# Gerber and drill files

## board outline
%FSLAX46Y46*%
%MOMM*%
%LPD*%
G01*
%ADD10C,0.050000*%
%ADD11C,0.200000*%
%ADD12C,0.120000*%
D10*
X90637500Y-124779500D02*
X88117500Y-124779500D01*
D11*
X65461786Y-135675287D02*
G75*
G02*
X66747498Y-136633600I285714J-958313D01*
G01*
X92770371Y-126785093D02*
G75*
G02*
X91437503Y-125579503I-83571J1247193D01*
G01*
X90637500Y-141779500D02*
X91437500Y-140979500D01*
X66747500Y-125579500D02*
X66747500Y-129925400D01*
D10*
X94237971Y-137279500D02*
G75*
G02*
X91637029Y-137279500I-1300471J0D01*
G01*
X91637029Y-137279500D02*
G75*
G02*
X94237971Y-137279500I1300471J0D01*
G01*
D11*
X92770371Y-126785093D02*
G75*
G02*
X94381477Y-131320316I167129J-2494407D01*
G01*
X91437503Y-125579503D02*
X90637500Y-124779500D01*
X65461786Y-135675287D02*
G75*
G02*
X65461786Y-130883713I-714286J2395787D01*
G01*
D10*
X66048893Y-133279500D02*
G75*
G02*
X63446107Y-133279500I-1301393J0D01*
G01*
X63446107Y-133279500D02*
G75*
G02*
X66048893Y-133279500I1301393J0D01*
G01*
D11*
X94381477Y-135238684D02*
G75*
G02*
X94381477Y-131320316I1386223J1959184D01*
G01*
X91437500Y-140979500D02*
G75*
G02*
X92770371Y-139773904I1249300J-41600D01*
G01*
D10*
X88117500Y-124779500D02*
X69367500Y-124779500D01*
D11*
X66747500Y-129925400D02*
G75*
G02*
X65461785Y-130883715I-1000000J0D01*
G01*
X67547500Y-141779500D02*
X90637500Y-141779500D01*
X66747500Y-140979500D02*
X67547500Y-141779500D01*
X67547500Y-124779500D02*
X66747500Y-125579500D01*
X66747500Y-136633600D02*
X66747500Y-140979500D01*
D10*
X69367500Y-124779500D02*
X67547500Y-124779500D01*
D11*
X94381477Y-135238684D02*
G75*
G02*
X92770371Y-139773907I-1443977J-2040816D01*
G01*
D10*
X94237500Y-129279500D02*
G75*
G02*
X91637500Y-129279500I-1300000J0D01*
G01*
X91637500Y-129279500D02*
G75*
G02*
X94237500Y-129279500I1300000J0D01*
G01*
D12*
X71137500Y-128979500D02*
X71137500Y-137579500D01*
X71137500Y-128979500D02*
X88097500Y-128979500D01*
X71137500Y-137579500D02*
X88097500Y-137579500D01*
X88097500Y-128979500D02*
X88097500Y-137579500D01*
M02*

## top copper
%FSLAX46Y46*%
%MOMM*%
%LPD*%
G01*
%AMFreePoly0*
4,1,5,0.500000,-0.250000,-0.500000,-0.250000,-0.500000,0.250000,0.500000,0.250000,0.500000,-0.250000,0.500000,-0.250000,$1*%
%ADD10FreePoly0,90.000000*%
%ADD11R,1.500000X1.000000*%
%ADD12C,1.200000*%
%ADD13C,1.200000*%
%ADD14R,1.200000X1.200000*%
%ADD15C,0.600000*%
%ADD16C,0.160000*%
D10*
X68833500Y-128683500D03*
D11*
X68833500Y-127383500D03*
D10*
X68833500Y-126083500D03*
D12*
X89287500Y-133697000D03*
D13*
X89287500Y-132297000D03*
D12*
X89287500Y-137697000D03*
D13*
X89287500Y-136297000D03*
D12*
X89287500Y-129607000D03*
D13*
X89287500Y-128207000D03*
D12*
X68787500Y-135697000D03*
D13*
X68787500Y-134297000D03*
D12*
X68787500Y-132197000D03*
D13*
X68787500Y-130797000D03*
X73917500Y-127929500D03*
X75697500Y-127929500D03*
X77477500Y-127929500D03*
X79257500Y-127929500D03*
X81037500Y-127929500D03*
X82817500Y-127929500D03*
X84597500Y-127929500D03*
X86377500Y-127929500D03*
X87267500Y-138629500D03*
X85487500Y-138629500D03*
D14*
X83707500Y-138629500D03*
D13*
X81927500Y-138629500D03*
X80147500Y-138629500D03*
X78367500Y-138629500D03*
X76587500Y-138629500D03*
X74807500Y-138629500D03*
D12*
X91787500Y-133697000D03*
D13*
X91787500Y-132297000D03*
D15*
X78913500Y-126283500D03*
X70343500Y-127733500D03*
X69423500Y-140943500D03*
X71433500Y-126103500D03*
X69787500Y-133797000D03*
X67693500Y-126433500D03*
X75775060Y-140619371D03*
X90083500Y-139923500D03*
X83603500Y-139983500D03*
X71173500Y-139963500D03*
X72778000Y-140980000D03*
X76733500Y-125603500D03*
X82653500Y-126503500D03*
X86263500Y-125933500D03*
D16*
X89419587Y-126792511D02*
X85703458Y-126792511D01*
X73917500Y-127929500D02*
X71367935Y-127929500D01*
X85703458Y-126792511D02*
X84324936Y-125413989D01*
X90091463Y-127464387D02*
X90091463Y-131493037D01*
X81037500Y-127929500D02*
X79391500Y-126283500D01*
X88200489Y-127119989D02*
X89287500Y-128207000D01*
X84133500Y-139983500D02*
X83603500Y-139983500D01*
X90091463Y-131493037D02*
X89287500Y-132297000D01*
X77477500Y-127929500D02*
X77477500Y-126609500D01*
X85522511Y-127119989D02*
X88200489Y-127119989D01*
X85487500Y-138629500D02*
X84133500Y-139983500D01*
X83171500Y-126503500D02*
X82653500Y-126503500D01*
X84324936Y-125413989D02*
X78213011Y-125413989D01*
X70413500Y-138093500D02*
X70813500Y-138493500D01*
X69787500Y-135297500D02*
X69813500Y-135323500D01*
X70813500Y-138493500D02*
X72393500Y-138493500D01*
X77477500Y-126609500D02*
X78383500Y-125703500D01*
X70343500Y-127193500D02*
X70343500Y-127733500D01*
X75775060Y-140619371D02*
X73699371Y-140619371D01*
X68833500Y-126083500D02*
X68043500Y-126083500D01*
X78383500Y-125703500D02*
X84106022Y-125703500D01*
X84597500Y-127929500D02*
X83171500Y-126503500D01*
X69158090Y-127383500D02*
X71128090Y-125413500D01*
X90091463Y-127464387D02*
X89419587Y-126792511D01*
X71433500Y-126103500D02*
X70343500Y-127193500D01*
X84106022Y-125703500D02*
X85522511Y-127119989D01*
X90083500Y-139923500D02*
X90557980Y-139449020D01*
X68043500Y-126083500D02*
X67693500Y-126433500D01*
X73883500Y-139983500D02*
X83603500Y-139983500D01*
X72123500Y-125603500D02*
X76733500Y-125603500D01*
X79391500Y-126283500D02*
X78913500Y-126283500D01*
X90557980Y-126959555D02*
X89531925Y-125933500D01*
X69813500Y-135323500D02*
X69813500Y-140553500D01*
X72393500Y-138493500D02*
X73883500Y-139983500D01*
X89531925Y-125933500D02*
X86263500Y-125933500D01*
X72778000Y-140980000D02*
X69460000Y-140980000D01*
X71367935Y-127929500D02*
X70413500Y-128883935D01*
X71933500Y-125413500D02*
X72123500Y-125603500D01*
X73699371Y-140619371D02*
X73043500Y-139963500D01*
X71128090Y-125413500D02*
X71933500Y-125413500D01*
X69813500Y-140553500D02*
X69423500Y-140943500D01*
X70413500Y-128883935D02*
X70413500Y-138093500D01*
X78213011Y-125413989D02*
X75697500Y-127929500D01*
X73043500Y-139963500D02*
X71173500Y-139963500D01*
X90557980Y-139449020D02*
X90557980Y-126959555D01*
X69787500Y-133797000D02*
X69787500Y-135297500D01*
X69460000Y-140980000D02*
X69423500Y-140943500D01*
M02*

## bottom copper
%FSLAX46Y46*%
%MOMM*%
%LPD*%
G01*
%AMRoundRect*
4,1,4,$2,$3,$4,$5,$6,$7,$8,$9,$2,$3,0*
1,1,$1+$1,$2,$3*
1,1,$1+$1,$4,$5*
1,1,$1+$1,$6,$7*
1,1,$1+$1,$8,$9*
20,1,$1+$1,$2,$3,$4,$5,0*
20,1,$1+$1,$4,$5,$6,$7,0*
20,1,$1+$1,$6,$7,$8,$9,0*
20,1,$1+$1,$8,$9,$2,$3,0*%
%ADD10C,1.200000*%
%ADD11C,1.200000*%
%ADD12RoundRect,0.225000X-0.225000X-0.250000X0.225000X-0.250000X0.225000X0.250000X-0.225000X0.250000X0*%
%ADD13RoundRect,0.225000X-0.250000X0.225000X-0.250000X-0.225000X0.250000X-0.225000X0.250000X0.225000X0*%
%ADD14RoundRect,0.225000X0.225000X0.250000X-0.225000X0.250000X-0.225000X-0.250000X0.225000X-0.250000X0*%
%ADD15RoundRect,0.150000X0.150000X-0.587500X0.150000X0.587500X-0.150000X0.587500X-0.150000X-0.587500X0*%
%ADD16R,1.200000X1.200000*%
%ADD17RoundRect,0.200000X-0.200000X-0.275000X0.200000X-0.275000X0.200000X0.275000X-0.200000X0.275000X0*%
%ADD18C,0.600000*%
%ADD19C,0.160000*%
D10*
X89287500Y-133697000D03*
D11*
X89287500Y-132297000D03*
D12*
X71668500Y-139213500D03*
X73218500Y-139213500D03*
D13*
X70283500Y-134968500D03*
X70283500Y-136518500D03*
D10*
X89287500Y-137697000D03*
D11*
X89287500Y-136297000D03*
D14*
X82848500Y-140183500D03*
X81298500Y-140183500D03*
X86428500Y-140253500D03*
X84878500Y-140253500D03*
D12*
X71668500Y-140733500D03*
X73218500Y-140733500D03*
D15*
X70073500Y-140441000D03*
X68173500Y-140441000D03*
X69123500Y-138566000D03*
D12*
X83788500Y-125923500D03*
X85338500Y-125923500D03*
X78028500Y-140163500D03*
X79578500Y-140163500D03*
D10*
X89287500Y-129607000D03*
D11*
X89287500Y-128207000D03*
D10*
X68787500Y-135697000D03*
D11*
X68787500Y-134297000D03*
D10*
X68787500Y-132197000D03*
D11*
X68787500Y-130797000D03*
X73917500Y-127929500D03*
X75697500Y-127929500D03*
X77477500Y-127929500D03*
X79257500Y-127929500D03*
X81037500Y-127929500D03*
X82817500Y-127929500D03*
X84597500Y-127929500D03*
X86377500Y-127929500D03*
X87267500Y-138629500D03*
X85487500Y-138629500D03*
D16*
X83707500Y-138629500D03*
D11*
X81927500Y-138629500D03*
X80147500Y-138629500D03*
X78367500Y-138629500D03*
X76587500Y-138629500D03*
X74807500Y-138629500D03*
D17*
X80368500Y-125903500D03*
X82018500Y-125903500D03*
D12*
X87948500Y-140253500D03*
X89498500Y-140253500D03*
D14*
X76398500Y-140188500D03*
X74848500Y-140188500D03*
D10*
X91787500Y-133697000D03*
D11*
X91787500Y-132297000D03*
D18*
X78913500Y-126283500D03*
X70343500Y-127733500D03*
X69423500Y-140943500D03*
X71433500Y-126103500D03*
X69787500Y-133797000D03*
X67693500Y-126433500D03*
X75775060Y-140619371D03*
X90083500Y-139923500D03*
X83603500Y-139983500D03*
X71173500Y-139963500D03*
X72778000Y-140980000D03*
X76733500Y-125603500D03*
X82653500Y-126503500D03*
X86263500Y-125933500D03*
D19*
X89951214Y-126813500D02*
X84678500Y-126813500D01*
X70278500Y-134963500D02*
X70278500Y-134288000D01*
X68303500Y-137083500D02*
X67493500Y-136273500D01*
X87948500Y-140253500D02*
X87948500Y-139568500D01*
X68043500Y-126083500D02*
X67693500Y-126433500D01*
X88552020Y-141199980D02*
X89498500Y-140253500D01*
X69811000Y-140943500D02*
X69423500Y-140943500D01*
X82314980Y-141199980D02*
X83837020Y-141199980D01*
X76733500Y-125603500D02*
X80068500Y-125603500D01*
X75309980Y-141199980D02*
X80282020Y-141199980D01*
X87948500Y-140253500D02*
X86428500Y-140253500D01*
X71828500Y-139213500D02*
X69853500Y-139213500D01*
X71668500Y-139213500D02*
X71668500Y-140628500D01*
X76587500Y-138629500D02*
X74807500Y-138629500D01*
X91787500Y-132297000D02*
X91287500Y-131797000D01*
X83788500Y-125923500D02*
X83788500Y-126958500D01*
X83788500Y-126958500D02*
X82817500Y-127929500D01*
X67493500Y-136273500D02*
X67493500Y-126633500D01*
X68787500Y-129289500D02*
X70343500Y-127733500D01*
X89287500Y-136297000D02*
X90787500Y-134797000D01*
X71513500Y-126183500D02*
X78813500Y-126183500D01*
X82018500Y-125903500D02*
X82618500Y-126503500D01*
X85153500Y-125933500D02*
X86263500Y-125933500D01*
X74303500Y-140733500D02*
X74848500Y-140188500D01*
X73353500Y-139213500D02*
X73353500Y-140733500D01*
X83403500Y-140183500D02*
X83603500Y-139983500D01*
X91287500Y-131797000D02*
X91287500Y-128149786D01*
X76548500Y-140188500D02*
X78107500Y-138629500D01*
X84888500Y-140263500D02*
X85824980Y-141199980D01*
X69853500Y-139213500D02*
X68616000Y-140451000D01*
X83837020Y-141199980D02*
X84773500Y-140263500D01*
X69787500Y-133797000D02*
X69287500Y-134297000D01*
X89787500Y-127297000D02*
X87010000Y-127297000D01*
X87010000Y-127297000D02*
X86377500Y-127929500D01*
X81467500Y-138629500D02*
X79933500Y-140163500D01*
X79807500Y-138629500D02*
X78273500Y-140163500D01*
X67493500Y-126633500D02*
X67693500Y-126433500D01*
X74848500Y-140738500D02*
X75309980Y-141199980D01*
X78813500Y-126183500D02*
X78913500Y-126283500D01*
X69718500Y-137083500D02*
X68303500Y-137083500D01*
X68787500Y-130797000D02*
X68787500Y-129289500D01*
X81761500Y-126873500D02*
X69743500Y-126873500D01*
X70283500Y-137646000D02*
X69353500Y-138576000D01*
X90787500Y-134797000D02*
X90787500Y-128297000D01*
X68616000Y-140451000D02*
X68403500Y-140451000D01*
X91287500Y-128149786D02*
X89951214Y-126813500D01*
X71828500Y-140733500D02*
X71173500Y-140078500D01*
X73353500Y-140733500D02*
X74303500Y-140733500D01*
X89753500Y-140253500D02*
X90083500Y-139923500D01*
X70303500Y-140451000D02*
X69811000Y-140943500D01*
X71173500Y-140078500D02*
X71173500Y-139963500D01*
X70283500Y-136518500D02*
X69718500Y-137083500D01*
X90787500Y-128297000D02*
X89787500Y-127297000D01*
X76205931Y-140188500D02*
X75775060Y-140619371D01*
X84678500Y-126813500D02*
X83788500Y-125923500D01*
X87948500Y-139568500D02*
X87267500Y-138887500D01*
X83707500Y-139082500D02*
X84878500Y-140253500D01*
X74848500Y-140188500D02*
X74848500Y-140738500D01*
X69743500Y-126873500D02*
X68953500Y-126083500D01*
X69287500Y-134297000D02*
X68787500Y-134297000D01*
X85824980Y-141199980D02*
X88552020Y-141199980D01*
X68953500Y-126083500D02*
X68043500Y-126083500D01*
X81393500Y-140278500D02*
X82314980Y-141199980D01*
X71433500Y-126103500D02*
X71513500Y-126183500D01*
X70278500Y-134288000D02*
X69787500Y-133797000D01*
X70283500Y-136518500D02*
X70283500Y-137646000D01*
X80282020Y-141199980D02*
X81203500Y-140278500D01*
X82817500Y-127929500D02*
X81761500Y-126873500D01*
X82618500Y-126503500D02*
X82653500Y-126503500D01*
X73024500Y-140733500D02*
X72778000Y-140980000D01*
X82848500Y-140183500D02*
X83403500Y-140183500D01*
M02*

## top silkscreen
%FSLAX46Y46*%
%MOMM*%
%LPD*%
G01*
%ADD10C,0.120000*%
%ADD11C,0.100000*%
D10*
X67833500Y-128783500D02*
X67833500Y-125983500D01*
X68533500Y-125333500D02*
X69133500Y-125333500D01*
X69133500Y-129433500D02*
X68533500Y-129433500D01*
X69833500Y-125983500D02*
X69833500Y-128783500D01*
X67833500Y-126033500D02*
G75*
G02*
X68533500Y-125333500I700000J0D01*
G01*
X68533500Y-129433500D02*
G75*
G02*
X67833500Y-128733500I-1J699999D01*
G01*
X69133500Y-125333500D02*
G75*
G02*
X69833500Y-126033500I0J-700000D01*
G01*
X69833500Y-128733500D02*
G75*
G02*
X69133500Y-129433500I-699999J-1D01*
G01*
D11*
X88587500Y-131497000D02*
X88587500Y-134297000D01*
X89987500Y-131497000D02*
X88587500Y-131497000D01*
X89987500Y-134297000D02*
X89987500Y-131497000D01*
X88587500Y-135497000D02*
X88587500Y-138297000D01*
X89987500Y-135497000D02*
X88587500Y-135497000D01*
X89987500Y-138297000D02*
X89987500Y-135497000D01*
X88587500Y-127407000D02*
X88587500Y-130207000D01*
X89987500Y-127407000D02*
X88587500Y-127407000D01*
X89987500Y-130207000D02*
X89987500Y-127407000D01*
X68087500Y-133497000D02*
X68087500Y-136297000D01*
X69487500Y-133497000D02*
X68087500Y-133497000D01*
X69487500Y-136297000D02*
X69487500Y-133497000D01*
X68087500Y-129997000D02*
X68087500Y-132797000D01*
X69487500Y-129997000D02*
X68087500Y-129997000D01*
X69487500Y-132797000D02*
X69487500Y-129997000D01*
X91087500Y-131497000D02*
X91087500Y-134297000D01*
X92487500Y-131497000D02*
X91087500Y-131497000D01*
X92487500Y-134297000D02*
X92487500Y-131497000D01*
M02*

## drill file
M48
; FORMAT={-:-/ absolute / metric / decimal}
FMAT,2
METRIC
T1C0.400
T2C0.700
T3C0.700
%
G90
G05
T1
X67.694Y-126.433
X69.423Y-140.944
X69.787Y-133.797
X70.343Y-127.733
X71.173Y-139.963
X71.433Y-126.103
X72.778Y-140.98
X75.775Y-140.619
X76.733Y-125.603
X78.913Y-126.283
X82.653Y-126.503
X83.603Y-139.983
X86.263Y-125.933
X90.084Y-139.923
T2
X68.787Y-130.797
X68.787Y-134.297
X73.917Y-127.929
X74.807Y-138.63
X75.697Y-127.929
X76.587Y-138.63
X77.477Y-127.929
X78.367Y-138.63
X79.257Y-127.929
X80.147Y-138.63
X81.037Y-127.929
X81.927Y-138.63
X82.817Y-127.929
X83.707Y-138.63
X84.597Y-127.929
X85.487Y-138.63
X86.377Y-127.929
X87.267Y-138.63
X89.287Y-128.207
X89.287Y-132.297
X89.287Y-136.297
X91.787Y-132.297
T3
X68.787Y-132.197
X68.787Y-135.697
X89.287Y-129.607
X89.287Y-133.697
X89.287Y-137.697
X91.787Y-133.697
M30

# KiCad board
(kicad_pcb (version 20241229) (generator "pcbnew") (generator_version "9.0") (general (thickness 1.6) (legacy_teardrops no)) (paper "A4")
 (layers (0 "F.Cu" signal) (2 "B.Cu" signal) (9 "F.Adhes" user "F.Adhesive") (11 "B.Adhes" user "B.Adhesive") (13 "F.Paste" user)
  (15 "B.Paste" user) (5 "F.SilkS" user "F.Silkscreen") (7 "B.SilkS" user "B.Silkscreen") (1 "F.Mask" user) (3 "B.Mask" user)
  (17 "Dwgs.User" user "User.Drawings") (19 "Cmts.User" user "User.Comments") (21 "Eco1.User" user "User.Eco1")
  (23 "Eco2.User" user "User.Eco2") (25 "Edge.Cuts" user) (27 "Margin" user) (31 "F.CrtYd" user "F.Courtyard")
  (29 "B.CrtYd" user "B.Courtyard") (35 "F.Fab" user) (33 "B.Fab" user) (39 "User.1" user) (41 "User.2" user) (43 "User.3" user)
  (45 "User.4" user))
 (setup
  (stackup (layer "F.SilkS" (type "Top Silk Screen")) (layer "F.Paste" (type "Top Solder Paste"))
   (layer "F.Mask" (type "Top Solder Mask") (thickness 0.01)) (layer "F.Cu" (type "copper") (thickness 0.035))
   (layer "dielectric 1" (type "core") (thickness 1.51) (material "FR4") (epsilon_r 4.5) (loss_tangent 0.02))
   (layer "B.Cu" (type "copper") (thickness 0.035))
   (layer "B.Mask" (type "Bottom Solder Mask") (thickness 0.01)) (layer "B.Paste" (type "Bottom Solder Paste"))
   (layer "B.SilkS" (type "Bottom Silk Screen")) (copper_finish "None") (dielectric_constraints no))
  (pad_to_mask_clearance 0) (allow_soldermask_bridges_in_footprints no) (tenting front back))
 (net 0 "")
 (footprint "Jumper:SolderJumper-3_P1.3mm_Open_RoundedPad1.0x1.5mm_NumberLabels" (layer "F.Cu") (at 68.8335 127.3835 90)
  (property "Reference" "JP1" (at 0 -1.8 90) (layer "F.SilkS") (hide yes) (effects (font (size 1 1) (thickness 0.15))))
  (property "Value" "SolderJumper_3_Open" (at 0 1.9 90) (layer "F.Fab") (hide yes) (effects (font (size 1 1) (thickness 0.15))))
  (fp_line (start -1.4 -1) (end 1.4 -1) (stroke (width 0.12) (type solid)) (layer "F.SilkS"))
  (fp_line (start 2.05 -0.3) (end 2.05 0.3) (stroke (width 0.12) (type solid)) (layer "F.SilkS"))
  (fp_line (start -2.05 0.3) (end -2.05 -0.3) (stroke (width 0.12) (type solid)) (layer "F.SilkS"))
  (fp_line (start 1.4 1) (end -1.4 1) (stroke (width 0.12) (type solid)) (layer "F.SilkS"))
  (fp_arc (start 1.35 -1) (mid 1.844975 -0.794975) (end 2.05 -0.3) (stroke (width 0.12) (type solid)) (layer "F.SilkS"))
  (fp_arc (start -2.05 -0.3) (mid -1.844975 -0.794975) (end -1.35 -1) (stroke (width 0.12) (type solid)) (layer "F.SilkS"))
  (fp_arc (start 2.05 0.3) (mid 1.844975 0.794975) (end 1.35 1) (stroke (width 0.12) (type solid)) (layer "F.SilkS"))
  (fp_arc (start -1.35 1) (mid -1.844975 0.794975) (end -2.05 0.3) (stroke (width 0.12) (type solid)) (layer "F.SilkS"))
  (pad "1" smd custom (at -1.3 0 90) (size 1 0.5) (layers "F.Cu" "F.Mask") (zone_connect 2) (options (clearance outline) (anchor rect))
   (primitives))
  (pad "2" smd rect (at 0 0 90) (size 1 1.5) (layers "F.Cu" "F.Mask"))
  (pad "3" smd custom (at 1.3 0 90) (size 1 0.5) (layers "F.Cu" "F.Mask") (zone_connect 2) (options (clearance outline) (anchor rect))
   (primitives)))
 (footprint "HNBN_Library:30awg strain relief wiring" (layer "B.Cu") (at 89.2875 132.297 90)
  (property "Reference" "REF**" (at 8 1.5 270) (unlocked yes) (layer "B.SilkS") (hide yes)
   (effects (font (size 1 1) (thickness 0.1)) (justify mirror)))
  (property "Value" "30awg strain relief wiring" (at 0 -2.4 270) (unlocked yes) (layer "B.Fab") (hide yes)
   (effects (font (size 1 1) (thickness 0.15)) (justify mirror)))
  (fp_line (start 0.8 -0.7) (end -2 -0.7) (stroke (width 0.1) (type default)) (layer "F.SilkS"))
  (fp_line (start 0.8 0.7) (end 0.8 -0.7) (stroke (width 0.1) (type default)) (layer "F.SilkS"))
  (fp_line (start -2 0.7) (end 0.8 0.7) (stroke (width 0.1) (type default)) (layer "F.SilkS"))
  (pad "" np_thru_hole circle (at -1.4 0 90) (size 1.2 1.2) (drill 0.7) (layers "*.Cu" "*.Mask")
   (teardrops (best_length_ratio 0.5) (max_length 1) (best_width_ratio 0.6) (max_width 2) (curved_edges no) (filter_ratio 0.9) (enabled no)
    (allow_two_segments yes) (prefer_zone_connections yes)))
  (pad "1" thru_hole circle (at 0 0 90) (size 1.2 1.2) (drill 0.7) (layers "*.Cu" "*.Mask") (remove_unused_layers no)))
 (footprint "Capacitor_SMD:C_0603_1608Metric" (layer "B.Cu") (at 72.4435 139.2135)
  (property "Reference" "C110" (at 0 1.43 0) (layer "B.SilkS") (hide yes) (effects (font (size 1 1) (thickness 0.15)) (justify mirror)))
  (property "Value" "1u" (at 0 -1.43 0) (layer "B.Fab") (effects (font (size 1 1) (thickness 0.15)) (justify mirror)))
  (pad "1" smd roundrect (at -0.775 0) (size 0.9 0.95) (layers "B.Cu" "B.Mask" "B.Paste") (roundrect_rratio 0.25))
  (pad "2" smd roundrect (at 0.775 0) (size 0.9 0.95) (layers "B.Cu" "B.Mask" "B.Paste") (roundrect_rratio 0.25)))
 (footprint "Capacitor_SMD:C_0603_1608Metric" (layer "B.Cu") (at 70.2835 135.7435 -90)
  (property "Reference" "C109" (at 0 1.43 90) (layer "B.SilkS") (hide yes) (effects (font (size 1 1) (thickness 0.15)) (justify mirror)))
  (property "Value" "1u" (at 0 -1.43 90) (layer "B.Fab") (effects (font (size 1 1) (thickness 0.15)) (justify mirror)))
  (pad "1" smd roundrect (at -0.775 0 270) (size 0.9 0.95) (layers "B.Cu" "B.Mask" "B.Paste") (roundrect_rratio 0.25))
  (pad "2" smd roundrect (at 0.775 0 270) (size 0.9 0.95) (layers "B.Cu" "B.Mask" "B.Paste") (roundrect_rratio 0.25)))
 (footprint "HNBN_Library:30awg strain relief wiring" (layer "B.Cu") (at 89.2875 136.297 90)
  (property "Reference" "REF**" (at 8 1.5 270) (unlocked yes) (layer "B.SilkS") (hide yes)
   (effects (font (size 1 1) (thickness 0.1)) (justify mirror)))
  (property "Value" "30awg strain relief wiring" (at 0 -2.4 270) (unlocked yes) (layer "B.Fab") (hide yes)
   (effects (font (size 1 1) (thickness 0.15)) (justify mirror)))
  (fp_line (start 0.8 -0.7) (end -2 -0.7) (stroke (width 0.1) (type default)) (layer "F.SilkS"))
  (fp_line (start 0.8 0.7) (end 0.8 -0.7) (stroke (width 0.1) (type default)) (layer "F.SilkS"))
  (fp_line (start -2 0.7) (end 0.8 0.7) (stroke (width 0.1) (type default)) (layer "F.SilkS"))
  (pad "" np_thru_hole circle (at -1.4 0 90) (size 1.2 1.2) (drill 0.7) (layers "*.Cu" "*.Mask")
   (teardrops (best_length_ratio 0.5) (max_length 1) (best_width_ratio 0.6) (max_width 2) (curved_edges no) (filter_ratio 0.9) (enabled no)
    (allow_two_segments yes) (prefer_zone_connections yes)))
  (pad "1" thru_hole circle (at 0 0 90) (size 1.2 1.2) (drill 0.7) (layers "*.Cu" "*.Mask") (remove_unused_layers no)))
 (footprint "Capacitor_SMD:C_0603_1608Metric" (layer "B.Cu") (at 82.0735 140.1835 180)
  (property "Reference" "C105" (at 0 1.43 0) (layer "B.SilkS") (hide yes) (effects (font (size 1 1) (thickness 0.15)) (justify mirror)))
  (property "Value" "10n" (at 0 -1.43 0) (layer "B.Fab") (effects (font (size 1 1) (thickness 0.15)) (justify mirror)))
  (pad "1" smd roundrect (at -0.775 0 180) (size 0.9 0.95) (layers "B.Cu" "B.Mask" "B.Paste") (roundrect_rratio 0.25))
  (pad "2" smd roundrect (at 0.775 0 180) (size 0.9 0.95) (layers "B.Cu" "B.Mask" "B.Paste") (roundrect_rratio 0.25)))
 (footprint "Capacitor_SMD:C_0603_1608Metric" (layer "B.Cu") (at 85.6535 140.2535 180)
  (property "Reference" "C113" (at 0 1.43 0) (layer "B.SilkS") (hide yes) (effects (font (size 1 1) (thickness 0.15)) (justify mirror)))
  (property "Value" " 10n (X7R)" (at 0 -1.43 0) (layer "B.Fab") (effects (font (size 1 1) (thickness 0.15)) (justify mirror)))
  (pad "1" smd roundrect (at -0.775 0 180) (size 0.9 0.95) (layers "B.Cu" "B.Mask" "B.Paste") (roundrect_rratio 0.25))
  (pad "2" smd roundrect (at 0.775 0 180) (size 0.9 0.95) (layers "B.Cu" "B.Mask" "B.Paste") (roundrect_rratio 0.25)))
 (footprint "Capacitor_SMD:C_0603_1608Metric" (layer "B.Cu") (at 72.4435 140.7335)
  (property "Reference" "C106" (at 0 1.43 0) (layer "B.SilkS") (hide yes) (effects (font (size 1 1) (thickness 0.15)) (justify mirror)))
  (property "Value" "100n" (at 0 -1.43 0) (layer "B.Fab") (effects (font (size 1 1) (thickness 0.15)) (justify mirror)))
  (pad "1" smd roundrect (at -0.775 0) (size 0.9 0.95) (layers "B.Cu" "B.Mask" "B.Paste") (roundrect_rratio 0.25))
  (pad "2" smd roundrect (at 0.775 0) (size 0.9 0.95) (layers "B.Cu" "B.Mask" "B.Paste") (roundrect_rratio 0.25)))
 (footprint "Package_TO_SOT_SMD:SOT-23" (layer "B.Cu") (at 69.1235 139.5035 90)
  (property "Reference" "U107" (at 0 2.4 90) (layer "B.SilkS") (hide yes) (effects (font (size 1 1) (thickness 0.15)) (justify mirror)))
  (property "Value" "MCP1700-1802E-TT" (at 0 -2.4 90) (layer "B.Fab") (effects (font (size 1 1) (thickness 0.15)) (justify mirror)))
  (pad "1" smd roundrect (at -0.9375 0.95 90) (size 1.475 0.6) (layers "B.Cu" "B.Mask" "B.Paste") (roundrect_rratio 0.25))
  (pad "2" smd roundrect (at -0.9375 -0.95 90) (size 1.475 0.6) (layers "B.Cu" "B.Mask" "B.Paste") (roundrect_rratio 0.25))
  (pad "3" smd roundrect (at 0.9375 0 90) (size 1.475 0.6) (layers "B.Cu" "B.Mask" "B.Paste") (roundrect_rratio 0.25)))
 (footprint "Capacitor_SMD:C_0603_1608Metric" (layer "B.Cu") (at 84.5635 125.9235)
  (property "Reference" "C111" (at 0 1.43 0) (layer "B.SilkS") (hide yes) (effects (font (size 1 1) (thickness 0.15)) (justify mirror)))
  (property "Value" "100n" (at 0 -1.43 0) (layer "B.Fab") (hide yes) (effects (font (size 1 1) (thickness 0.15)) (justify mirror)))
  (pad "1" smd roundrect (at -0.775 0) (size 0.9 0.95) (layers "B.Cu" "B.Mask" "B.Paste") (roundrect_rratio 0.25))
  (pad "2" smd roundrect (at 0.775 0) (size 0.9 0.95) (layers "B.Cu" "B.Mask" "B.Paste") (roundrect_rratio 0.25)))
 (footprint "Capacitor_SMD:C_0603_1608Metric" (layer "B.Cu") (at 78.8035 140.1635)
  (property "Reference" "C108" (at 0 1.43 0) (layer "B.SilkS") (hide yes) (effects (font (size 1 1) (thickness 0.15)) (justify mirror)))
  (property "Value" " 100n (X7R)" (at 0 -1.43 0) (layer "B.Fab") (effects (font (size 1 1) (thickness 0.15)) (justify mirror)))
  (pad "1" smd roundrect (at -0.775 0) (size 0.9 0.95) (layers "B.Cu" "B.Mask" "B.Paste") (roundrect_rratio 0.25))
  (pad "2" smd roundrect (at 0.775 0) (size 0.9 0.95) (layers "B.Cu" "B.Mask" "B.Paste") (roundrect_rratio 0.25)))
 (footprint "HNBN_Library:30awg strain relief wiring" (layer "B.Cu") (at 89.2875 128.207 90)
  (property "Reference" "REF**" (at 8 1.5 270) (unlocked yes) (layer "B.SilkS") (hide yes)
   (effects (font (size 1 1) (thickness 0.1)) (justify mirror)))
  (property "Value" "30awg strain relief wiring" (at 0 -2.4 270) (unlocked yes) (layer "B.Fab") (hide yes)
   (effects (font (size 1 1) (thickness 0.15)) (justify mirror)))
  (fp_line (start 0.8 -0.7) (end -2 -0.7) (stroke (width 0.1) (type default)) (layer "F.SilkS"))
  (fp_line (start 0.8 0.7) (end 0.8 -0.7) (stroke (width 0.1) (type default)) (layer "F.SilkS"))
  (fp_line (start -2 0.7) (end 0.8 0.7) (stroke (width 0.1) (type default)) (layer "F.SilkS"))
  (pad "" np_thru_hole circle (at -1.4 0 90) (size 1.2 1.2) (drill 0.7) (layers "*.Cu" "*.Mask")
   (teardrops (best_length_ratio 0.5) (max_length 1) (best_width_ratio 0.6) (max_width 2) (curved_edges no) (filter_ratio 0.9) (enabled no)
    (allow_two_segments yes) (prefer_zone_connections yes)))
  (pad "1" thru_hole circle (at 0 0 90) (size 1.2 1.2) (drill 0.7) (layers "*.Cu" "*.Mask") (remove_unused_layers no)))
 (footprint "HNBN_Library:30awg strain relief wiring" (layer "B.Cu") (at 68.7875 134.297 90)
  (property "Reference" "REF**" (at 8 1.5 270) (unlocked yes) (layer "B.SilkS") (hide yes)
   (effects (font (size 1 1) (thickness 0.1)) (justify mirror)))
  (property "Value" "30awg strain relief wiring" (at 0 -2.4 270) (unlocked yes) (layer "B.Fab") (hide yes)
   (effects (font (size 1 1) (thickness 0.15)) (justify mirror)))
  (fp_line (start 0.8 -0.7) (end -2 -0.7) (stroke (width 0.1) (type default)) (layer "F.SilkS"))
  (fp_line (start 0.8 0.7) (end 0.8 -0.7) (stroke (width 0.1) (type default)) (layer "F.SilkS"))
  (fp_line (start -2 0.7) (end 0.8 0.7) (stroke (width 0.1) (type default)) (layer "F.SilkS"))
  (pad "" np_thru_hole circle (at -1.4 0 90) (size 1.2 1.2) (drill 0.7) (layers "*.Cu" "*.Mask")
   (teardrops (best_length_ratio 0.5) (max_length 1) (best_width_ratio 0.6) (max_width 2) (curved_edges no) (filter_ratio 0.9) (enabled no)
    (allow_two_segments yes) (prefer_zone_connections yes)))
  (pad "1" thru_hole circle (at 0 0 90) (size 1.2 1.2) (drill 0.7) (layers "*.Cu" "*.Mask") (remove_unused_layers no)))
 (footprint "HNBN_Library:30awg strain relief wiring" (layer "B.Cu") (at 68.7875 130.797 90)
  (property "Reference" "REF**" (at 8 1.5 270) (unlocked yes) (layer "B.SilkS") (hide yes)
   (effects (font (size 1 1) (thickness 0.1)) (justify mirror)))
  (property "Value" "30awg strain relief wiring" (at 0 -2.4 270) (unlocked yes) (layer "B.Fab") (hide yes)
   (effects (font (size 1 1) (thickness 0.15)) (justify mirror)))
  (fp_line (start 0.8 -0.7) (end -2 -0.7) (stroke (width 0.1) (type default)) (layer "F.SilkS"))
  (fp_line (start 0.8 0.7) (end 0.8 -0.7) (stroke (width 0.1) (type default)) (layer "F.SilkS"))
  (fp_line (start -2 0.7) (end 0.8 0.7) (stroke (width 0.1) (type default)) (layer "F.SilkS"))
  (pad "" np_thru_hole circle (at -1.4 0 90) (size 1.2 1.2) (drill 0.7) (layers "*.Cu" "*.Mask")
   (teardrops (best_length_ratio 0.5) (max_length 1) (best_width_ratio 0.6) (max_width 2) (curved_edges no) (filter_ratio 0.9) (enabled no)
    (allow_two_segments yes) (prefer_zone_connections yes)))
  (pad "1" thru_hole circle (at 0 0 90) (size 1.2 1.2) (drill 0.7) (layers "*.Cu" "*.Mask") (remove_unused_layers no)))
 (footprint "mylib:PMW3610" (layer "B.Cu") (at 73.9175 127.9295 -90)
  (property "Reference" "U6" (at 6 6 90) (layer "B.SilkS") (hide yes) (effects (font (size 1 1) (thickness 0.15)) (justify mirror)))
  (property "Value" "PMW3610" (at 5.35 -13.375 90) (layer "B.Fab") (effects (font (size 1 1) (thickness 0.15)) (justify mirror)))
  (fp_line (start 1.05 2.78) (end 9.65 2.78) (stroke (width 0.12) (type solid)) (layer "Edge.Cuts"))
  (fp_line (start 1.05 2.78) (end 1.05 -14.18) (stroke (width 0.12) (type solid)) (layer "Edge.Cuts"))
  (fp_line (start 9.65 2.78) (end 9.65 -14.18) (stroke (width 0.12) (type solid)) (layer "Edge.Cuts"))
  (fp_line (start 1.05 -14.18) (end 9.65 -14.18) (stroke (width 0.12) (type solid)) (layer "Edge.Cuts"))
  (pad "1" thru_hole circle (at 0 0 270) (size 1.2 1.2) (drill 0.7) (layers "*.Cu" "*.Mask") (remove_unused_layers no))
  (pad "2" thru_hole circle (at 0 -1.78 270) (size 1.2 1.2) (drill 0.7) (layers "*.Cu" "*.Mask") (remove_unused_layers no))
  (pad "3" thru_hole circle (at 0 -3.56 270) (size 1.2 1.2) (drill 0.7) (layers "*.Cu" "*.Mask") (remove_unused_layers no))
  (pad "4" thru_hole circle (at 0 -5.34 270) (size 1.2 1.2) (drill 0.7) (layers "*.Cu" "*.Mask") (remove_unused_layers no))
  (pad "5" thru_hole circle (at 0 -7.12 270) (size 1.2 1.2) (drill 0.7) (layers "*.Cu" "*.Mask") (remove_unused_layers no))
  (pad "6" thru_hole circle (at 0 -8.9 270) (size 1.2 1.2) (drill 0.7) (layers "*.Cu" "*.Mask") (remove_unused_layers no))
  (pad "7" thru_hole circle (at 0 -10.68 270) (size 1.2 1.2) (drill 0.7) (layers "*.Cu" "*.Mask") (remove_unused_layers no))
  (pad "8" thru_hole circle (at 0 -12.46 270) (size 1.2 1.2) (drill 0.7) (layers "*.Cu" "*.Mask") (remove_unused_layers no))
  (pad "9" thru_hole circle (at 10.7 -13.35 270) (size 1.2 1.2) (drill 0.7) (layers "*.Cu" "*.Mask") (remove_unused_layers no))
  (pad "10" thru_hole circle (at 10.7 -11.57 270) (size 1.2 1.2) (drill 0.7) (layers "*.Cu" "*.Mask") (remove_unused_layers no))
  (pad "11" thru_hole rect (at 10.7 -9.79 270) (size 1.2 1.2) (drill 0.7) (layers "*.Cu" "*.Mask") (remove_unused_layers no))
  (pad "12" thru_hole circle (at 10.7 -8.01 270) (size 1.2 1.2) (drill 0.7) (layers "*.Cu" "*.Mask") (remove_unused_layers no))
  (pad "13" thru_hole circle (at 10.7 -6.23 270) (size 1.2 1.2) (drill 0.7) (layers "*.Cu" "*.Mask") (remove_unused_layers no))
  (pad "14" thru_hole circle (at 10.7 -4.45 270) (size 1.2 1.2) (drill 0.7) (layers "*.Cu" "*.Mask") (remove_unused_layers no))
  (pad "15" thru_hole circle (at 10.7 -2.67 270) (size 1.2 1.2) (drill 0.7) (layers "*.Cu" "*.Mask") (remove_unused_layers no))
  (pad "16" thru_hole circle (at 10.7 -0.89 270) (size 1.2 1.2) (drill 0.7) (layers "*.Cu" "*.Mask") (remove_unused_layers no)))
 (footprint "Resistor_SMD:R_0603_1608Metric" (layer "B.Cu") (at 81.1935 125.9035)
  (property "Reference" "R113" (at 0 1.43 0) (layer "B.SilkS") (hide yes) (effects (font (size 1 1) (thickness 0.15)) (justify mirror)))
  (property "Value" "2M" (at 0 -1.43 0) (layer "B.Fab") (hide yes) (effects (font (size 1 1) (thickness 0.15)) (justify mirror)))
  (pad "1" smd roundrect (at -0.825 0) (size 0.8 0.95) (layers "B.Cu" "B.Mask" "B.Paste") (roundrect_rratio 0.25))
  (pad "2" smd roundrect (at 0.825 0) (size 0.8 0.95) (layers "B.Cu" "B.Mask" "B.Paste") (roundrect_rratio 0.25)))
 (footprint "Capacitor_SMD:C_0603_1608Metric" (layer "B.Cu") (at 88.7235 140.2535)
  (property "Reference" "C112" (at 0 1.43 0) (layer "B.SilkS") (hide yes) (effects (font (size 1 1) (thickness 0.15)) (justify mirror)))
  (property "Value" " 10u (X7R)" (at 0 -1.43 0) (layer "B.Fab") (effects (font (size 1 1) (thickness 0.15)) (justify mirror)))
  (pad "1" smd roundrect (at -0.775 0) (size 0.9 0.95) (layers "B.Cu" "B.Mask" "B.Paste") (roundrect_rratio 0.25))
  (pad "2" smd roundrect (at 0.775 0) (size 0.9 0.95) (layers "B.Cu" "B.Mask" "B.Paste") (roundrect_rratio 0.25)))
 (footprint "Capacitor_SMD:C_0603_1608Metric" (layer "B.Cu") (at 75.6235 140.1885 180)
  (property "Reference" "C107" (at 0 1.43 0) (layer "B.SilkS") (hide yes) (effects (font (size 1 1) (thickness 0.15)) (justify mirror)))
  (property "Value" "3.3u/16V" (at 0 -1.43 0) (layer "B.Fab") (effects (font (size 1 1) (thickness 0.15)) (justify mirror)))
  (pad "1" smd roundrect (at -0.775 0 180) (size 0.9 0.95) (layers "B.Cu" "B.Mask" "B.Paste") (roundrect_rratio 0.25))
  (pad "2" smd roundrect (at 0.775 0 180) (size 0.9 0.95) (layers "B.Cu" "B.Mask" "B.Paste") (roundrect_rratio 0.25)))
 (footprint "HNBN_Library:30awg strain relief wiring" (layer "B.Cu") (at 91.7875 132.297 90)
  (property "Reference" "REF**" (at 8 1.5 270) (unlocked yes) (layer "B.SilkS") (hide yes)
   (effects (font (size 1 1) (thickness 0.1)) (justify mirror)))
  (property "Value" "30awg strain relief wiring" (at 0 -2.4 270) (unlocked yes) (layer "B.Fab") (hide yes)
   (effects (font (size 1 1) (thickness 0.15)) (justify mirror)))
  (fp_line (start 0.8 -0.7) (end -2 -0.7) (stroke (width 0.1) (type default)) (layer "F.SilkS"))
  (fp_line (start 0.8 0.7) (end 0.8 -0.7) (stroke (width 0.1) (type default)) (layer "F.SilkS"))
  (fp_line (start -2 0.7) (end 0.8 0.7) (stroke (width 0.1) (type default)) (layer "F.SilkS"))
  (pad "" np_thru_hole circle (at -1.4 0 90) (size 1.2 1.2) (drill 0.7) (layers "*.Cu" "*.Mask")
   (teardrops (best_length_ratio 0.5) (max_length 1) (best_width_ratio 0.6) (max_width 2) (curved_edges no) (filter_ratio 0.9) (enabled no)
    (allow_two_segments yes) (prefer_zone_connections yes)))
  (pad "1" thru_hole circle (at 0 0 90) (size 1.2 1.2) (drill 0.7) (layers "*.Cu" "*.Mask") (remove_unused_layers no)))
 (gr_line (start 90.6375 124.7795) (end 88.1175 124.7795) (stroke (width 0.05) (type default)) (layer "Edge.Cuts"))
 (gr_arc (start 65.461786 135.675287) (mid 66.345113 135.831818) (end 66.7475 136.6336) (stroke (width 0.2) (type default))
  (layer "Edge.Cuts"))
 (gr_arc (start 92.770371 126.785093) (mid 91.848295 126.464929) (end 91.437503 125.579503) (stroke (width 0.2) (type default))
  (layer "Edge.Cuts"))
 (gr_line (start 90.6375 141.7795) (end 91.4375 140.9795) (stroke (width 0.2) (type default)) (layer "Edge.Cuts"))
 (gr_line (start 66.7475 125.5795) (end 66.7475 129.9254) (stroke (width 0.2) (type default)) (layer "Edge.Cuts"))
 (gr_circle (center 92.9375 137.2795) (end 92.9025 135.9795) (stroke (width 0.05) (type default)) (fill no) (layer "Edge.Cuts"))
 (gr_arc (start 92.770371 126.785093) (mid 95.293269 128.44263) (end 94.381477 131.320316) (stroke (width 0.2) (type default))
  (layer "Edge.Cuts"))
 (gr_line (start 91.437503 125.579503) (end 90.6375 124.7795) (stroke (width 0.2) (type default)) (layer "Edge.Cuts"))
 (gr_arc (start 65.461786 135.675287) (mid 62.2475 133.2795) (end 65.461786 130.883713) (stroke (width 0.2) (type default))
  (layer "Edge.Cuts"))
 (gr_circle (center 64.7475 133.2795) (end 64.5125 131.9995) (stroke (width 0.05) (type default)) (fill no) (layer "Edge.Cuts"))
 (gr_arc (start 94.381477 135.238684) (mid 93.367697 133.2795) (end 94.381477 131.320316) (stroke (width 0.2) (type default))
  (layer "Edge.Cuts"))
 (gr_arc (start 91.4375 140.9795) (mid 91.848292 140.09407) (end 92.770371 139.773907) (stroke (width 0.2) (type default))
  (layer "Edge.Cuts"))
 (gr_line (start 88.1175 124.7795) (end 69.3675 124.7795) (stroke (width 0.05) (type default)) (layer "Edge.Cuts"))
 (gr_arc (start 66.7475 129.9254) (mid 66.345114 130.727184) (end 65.461786 130.883713) (stroke (width 0.2) (type default))
  (layer "Edge.Cuts"))
 (gr_line (start 67.5475 141.7795) (end 90.6375 141.7795) (stroke (width 0.2) (type default)) (layer "Edge.Cuts"))
 (gr_line (start 66.7475 140.9795) (end 67.5475 141.7795) (stroke (width 0.2) (type default)) (layer "Edge.Cuts"))
 (gr_line (start 67.5475 124.7795) (end 66.7475 125.5795) (stroke (width 0.2) (type default)) (layer "Edge.Cuts"))
 (gr_line (start 66.7475 136.6336) (end 66.7475 140.9795) (stroke (width 0.2) (type default)) (layer "Edge.Cuts"))
 (gr_line (start 69.3675 124.7795) (end 67.5475 124.7795) (stroke (width 0.05) (type default)) (layer "Edge.Cuts"))
 (gr_arc (start 94.381477 135.238684) (mid 95.293269 138.11637) (end 92.770371 139.773907) (stroke (width 0.2) (type default))
  (layer "Edge.Cuts"))
 (gr_circle (center 92.9375 129.2795) (end 92.9375 127.9795) (stroke (width 0.05) (type default)) (fill no) (layer "Edge.Cuts"))
 (segment (start 89.419587 126.792511) (end 85.703458 126.792511) (width 0.16) (layer "F.Cu") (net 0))
 (segment (start 73.9175 127.9295) (end 71.367935 127.9295) (width 0.16) (layer "F.Cu") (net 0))
 (segment (start 85.703458 126.792511) (end 84.324936 125.413989) (width 0.16) (layer "F.Cu") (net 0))
 (segment (start 90.091463 127.464387) (end 90.091463 131.493037) (width 0.16) (layer "F.Cu") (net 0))
 (segment (start 81.0375 127.9295) (end 79.3915 126.2835) (width 0.16) (layer "F.Cu") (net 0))
 (segment (start 88.200489 127.119989) (end 89.2875 128.207) (width 0.16) (layer "F.Cu") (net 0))
 (segment (start 84.1335 139.9835) (end 83.6035 139.9835) (width 0.16) (layer "F.Cu") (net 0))
 (segment (start 90.091463 131.493037) (end 89.2875 132.297) (width 0.16) (layer "F.Cu") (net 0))
 (segment (start 77.4775 127.9295) (end 77.4775 126.6095) (width 0.16) (layer "F.Cu") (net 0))
 (segment (start 85.522511 127.119989) (end 88.200489 127.119989) (width 0.16) (layer "F.Cu") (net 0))
 (segment (start 85.4875 138.6295) (end 84.1335 139.9835) (width 0.16) (layer "F.Cu") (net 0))
 (segment (start 83.1715 126.5035) (end 82.6535 126.5035) (width 0.16) (layer "F.Cu") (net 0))
 (segment (start 84.324936 125.413989) (end 78.213011 125.413989) (width 0.16) (layer "F.Cu") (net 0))
 (segment (start 70.4135 138.0935) (end 70.8135 138.4935) (width 0.16) (layer "F.Cu") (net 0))
 (segment (start 69.7875 135.2975) (end 69.8135 135.3235) (width 0.16) (layer "F.Cu") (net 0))
 (segment (start 70.8135 138.4935) (end 72.3935 138.4935) (width 0.16) (layer "F.Cu") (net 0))
 (segment (start 77.4775 126.6095) (end 78.3835 125.7035) (width 0.16) (layer "F.Cu") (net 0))
 (segment (start 70.3435 127.1935) (end 70.3435 127.7335) (width 0.16) (layer "F.Cu") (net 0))
 (segment (start 75.77506 140.619371) (end 73.699371 140.619371) (width 0.16) (layer "F.Cu") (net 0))
 (segment (start 68.8335 126.0835) (end 68.0435 126.0835) (width 0.16) (layer "F.Cu") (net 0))
 (segment (start 78.3835 125.7035) (end 84.106022 125.7035) (width 0.16) (layer "F.Cu") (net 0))
 (segment (start 84.5975 127.9295) (end 83.1715 126.5035) (width 0.16) (layer "F.Cu") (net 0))
 (segment (start 69.15809 127.3835) (end 71.12809 125.4135) (width 0.16) (layer "F.Cu") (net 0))
 (segment (start 90.091463 127.464387) (end 89.419587 126.792511) (width 0.16) (layer "F.Cu") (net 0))
 (segment (start 71.4335 126.1035) (end 70.3435 127.1935) (width 0.16) (layer "F.Cu") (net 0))
 (segment (start 84.106022 125.7035) (end 85.522511 127.119989) (width 0.16) (layer "F.Cu") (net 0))
 (segment (start 90.0835 139.9235) (end 90.55798 139.44902) (width 0.16) (layer "F.Cu") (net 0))
 (segment (start 68.0435 126.0835) (end 67.6935 126.4335) (width 0.16) (layer "F.Cu") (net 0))
 (segment (start 73.8835 139.9835) (end 83.6035 139.9835) (width 0.16) (layer "F.Cu") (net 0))
 (segment (start 72.1235 125.6035) (end 76.7335 125.6035) (width 0.16) (layer "F.Cu") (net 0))
 (segment (start 79.3915 126.2835) (end 78.9135 126.2835) (width 0.16) (layer "F.Cu") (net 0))
 (segment (start 90.55798 126.959555) (end 89.531925 125.9335) (width 0.16) (layer "F.Cu") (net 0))
 (segment (start 69.8135 135.3235) (end 69.8135 140.5535) (width 0.16) (layer "F.Cu") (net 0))
 (segment (start 72.3935 138.4935) (end 73.8835 139.9835) (width 0.16) (layer "F.Cu") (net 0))
 (segment (start 89.531925 125.9335) (end 86.2635 125.9335) (width 0.16) (layer "F.Cu") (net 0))
 (segment (start 72.778 140.98) (end 69.46 140.98) (width 0.16) (layer "F.Cu") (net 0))
 (segment (start 71.367935 127.9295) (end 70.4135 128.883935) (width 0.16) (layer "F.Cu") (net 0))
 (segment (start 71.9335 125.4135) (end 72.1235 125.6035) (width 0.16) (layer "F.Cu") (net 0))
 (segment (start 73.699371 140.619371) (end 73.0435 139.9635) (width 0.16) (layer "F.Cu") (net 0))
 (segment (start 71.12809 125.4135) (end 71.9335 125.4135) (width 0.16) (layer "F.Cu") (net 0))
 (segment (start 69.8135 140.5535) (end 69.4235 140.9435) (width 0.16) (layer "F.Cu") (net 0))
 (segment (start 70.4135 128.883935) (end 70.4135 138.0935) (width 0.16) (layer "F.Cu") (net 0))
 (segment (start 78.213011 125.413989) (end 75.6975 127.9295) (width 0.16) (layer "F.Cu") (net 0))
 (segment (start 73.0435 139.9635) (end 71.1735 139.9635) (width 0.16) (layer "F.Cu") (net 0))
 (segment (start 90.55798 139.44902) (end 90.55798 126.959555) (width 0.16) (layer "F.Cu") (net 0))
 (segment (start 69.7875 133.797) (end 69.7875 135.2975) (width 0.16) (layer "F.Cu") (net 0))
 (segment (start 69.46 140.98) (end 69.4235 140.9435) (width 0.16) (layer "F.Cu") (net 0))
 (via (at 78.9135 126.2835) (size 0.6) (drill 0.4) (layers "F.Cu" "B.Cu") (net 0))
 (via (at 70.3435 127.7335) (size 0.6) (drill 0.4) (layers "F.Cu" "B.Cu") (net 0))
 (via (at 69.4235 140.9435) (size 0.6) (drill 0.4) (layers "F.Cu" "B.Cu") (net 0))
 (via (at 71.4335 126.1035) (size 0.6) (drill 0.4) (layers "F.Cu" "B.Cu") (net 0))
 (via (at 69.7875 133.797) (size 0.6) (drill 0.4) (layers "F.Cu" "B.Cu") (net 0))
 (via (at 67.6935 126.4335) (size 0.6) (drill 0.4) (layers "F.Cu" "B.Cu") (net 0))
 (via (at 75.77506 140.619371) (size 0.6) (drill 0.4) (layers "F.Cu" "B.Cu") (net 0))
 (via (at 90.0835 139.9235) (size 0.6) (drill 0.4) (layers "F.Cu" "B.Cu") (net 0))
 (via (at 83.6035 139.9835) (size 0.6) (drill 0.4) (layers "F.Cu" "B.Cu") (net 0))
 (via (at 71.1735 139.9635) (size 0.6) (drill 0.4) (layers "F.Cu" "B.Cu") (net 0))
 (via (at 72.778 140.98) (size 0.6) (drill 0.4) (layers "F.Cu" "B.Cu") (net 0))
 (via (at 76.7335 125.6035) (size 0.6) (drill 0.4) (layers "F.Cu" "B.Cu") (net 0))
 (via (at 82.6535 126.5035) (size 0.6) (drill 0.4) (layers "F.Cu" "B.Cu") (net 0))
 (via (at 86.2635 125.9335) (size 0.6) (drill 0.4) (layers "F.Cu" "B.Cu") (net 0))
 (segment (start 89.951214 126.8135) (end 84.6785 126.8135) (width 0.16) (layer "B.Cu") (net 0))
 (segment (start 70.2785 134.9635) (end 70.2785 134.288) (width 0.16) (layer "B.Cu") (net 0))
 (segment (start 68.3035 137.0835) (end 67.4935 136.2735) (width 0.16) (layer "B.Cu") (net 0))
 (segment (start 87.9485 140.2535) (end 87.9485 139.5685) (width 0.16) (layer "B.Cu") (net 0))
 (segment (start 68.0435 126.0835) (end 67.6935 126.4335) (width 0.16) (layer "B.Cu") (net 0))
 (segment (start 88.55202 141.19998) (end 89.4985 140.2535) (width 0.16) (layer "B.Cu") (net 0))
 (segment (start 69.811 140.9435) (end 69.4235 140.9435) (width 0.16) (layer "B.Cu") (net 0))
 (segment (start 82.31498 141.19998) (end 83.83702 141.19998) (width 0.16) (layer "B.Cu") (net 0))
 (segment (start 76.7335 125.6035) (end 80.0685 125.6035) (width 0.16) (layer "B.Cu") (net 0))
 (segment (start 75.30998 141.19998) (end 80.28202 141.19998) (width 0.16) (layer "B.Cu") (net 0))
 (segment (start 87.9485 140.2535) (end 86.4285 140.2535) (width 0.16) (layer "B.Cu") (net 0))
 (segment (start 71.8285 139.2135) (end 69.8535 139.2135) (width 0.16) (layer "B.Cu") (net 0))
 (segment (start 71.6685 139.2135) (end 71.6685 140.6285) (width 0.16) (layer "B.Cu") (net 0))
 (segment (start 76.5875 138.6295) (end 74.8075 138.6295) (width 0.16) (layer "B.Cu") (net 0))
 (segment (start 91.7875 132.297) (end 91.2875 131.797) (width 0.16) (layer "B.Cu") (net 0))
 (segment (start 83.7885 125.9235) (end 83.7885 126.9585) (width 0.16) (layer "B.Cu") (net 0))
 (segment (start 83.7885 126.9585) (end 82.8175 127.9295) (width 0.16) (layer "B.Cu") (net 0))
 (segment (start 67.4935 136.2735) (end 67.4935 126.6335) (width 0.16) (layer "B.Cu") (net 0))
 (segment (start 68.7875 129.2895) (end 70.3435 127.7335) (width 0.16) (layer "B.Cu") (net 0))
 (segment (start 89.2875 136.297) (end 90.7875 134.797) (width 0.16) (layer "B.Cu") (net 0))
 (segment (start 71.5135 126.1835) (end 78.8135 126.1835) (width 0.16) (layer "B.Cu") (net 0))
 (segment (start 82.0185 125.9035) (end 82.6185 126.5035) (width 0.16) (layer "B.Cu") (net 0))
 (segment (start 85.1535 125.9335) (end 86.2635 125.9335) (width 0.16) (layer "B.Cu") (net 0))
 (segment (start 74.3035 140.7335) (end 74.8485 140.1885) (width 0.16) (layer "B.Cu") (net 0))
 (segment (start 73.3535 139.2135) (end 73.3535 140.7335) (width 0.16) (layer "B.Cu") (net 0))
 (segment (start 83.4035 140.1835) (end 83.6035 139.9835) (width 0.16) (layer "B.Cu") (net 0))
 (segment (start 91.2875 131.797) (end 91.2875 128.149786) (width 0.16) (layer "B.Cu") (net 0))
 (segment (start 76.5485 140.1885) (end 78.1075 138.6295) (width 0.16) (layer "B.Cu") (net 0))
 (segment (start 84.8885 140.2635) (end 85.82498 141.19998) (width 0.16) (layer "B.Cu") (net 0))
 (segment (start 69.8535 139.2135) (end 68.616 140.451) (width 0.16) (layer "B.Cu") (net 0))
 (segment (start 83.83702 141.19998) (end 84.7735 140.2635) (width 0.16) (layer "B.Cu") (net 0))
 (segment (start 69.7875 133.797) (end 69.2875 134.297) (width 0.16) (layer "B.Cu") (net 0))
 (segment (start 89.7875 127.297) (end 87.01 127.297) (width 0.16) (layer "B.Cu") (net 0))
 (segment (start 87.01 127.297) (end 86.3775 127.9295) (width 0.16) (layer "B.Cu") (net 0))
 (segment (start 81.4675 138.6295) (end 79.9335 140.1635) (width 0.16) (layer "B.Cu") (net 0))
 (segment (start 79.8075 138.6295) (end 78.2735 140.1635) (width 0.16) (layer "B.Cu") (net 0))
 (segment (start 67.4935 126.6335) (end 67.6935 126.4335) (width 0.16) (layer "B.Cu") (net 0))
 (segment (start 74.8485 140.7385) (end 75.30998 141.19998) (width 0.16) (layer "B.Cu") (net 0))
 (segment (start 78.8135 126.1835) (end 78.9135 126.2835) (width 0.16) (layer "B.Cu") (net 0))
 (segment (start 69.7185 137.0835) (end 68.3035 137.0835) (width 0.16) (layer "B.Cu") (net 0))
 (segment (start 68.7875 130.797) (end 68.7875 129.2895) (width 0.16) (layer "B.Cu") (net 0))
 (segment (start 81.7615 126.8735) (end 69.7435 126.8735) (width 0.16) (layer "B.Cu") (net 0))
 (segment (start 70.2835 137.646) (end 69.3535 138.576) (width 0.16) (layer "B.Cu") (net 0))
 (segment (start 90.7875 134.797) (end 90.7875 128.297) (width 0.16) (layer "B.Cu") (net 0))
 (segment (start 68.616 140.451) (end 68.4035 140.451) (width 0.16) (layer "B.Cu") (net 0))
 (segment (start 91.2875 128.149786) (end 89.951214 126.8135) (width 0.16) (layer "B.Cu") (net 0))
 (segment (start 71.8285 140.7335) (end 71.1735 140.0785) (width 0.16) (layer "B.Cu") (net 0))
 (segment (start 73.3535 140.7335) (end 74.3035 140.7335) (width 0.16) (layer "B.Cu") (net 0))
 (segment (start 89.7535 140.2535) (end 90.0835 139.9235) (width 0.16) (layer "B.Cu") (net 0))
 (segment (start 70.3035 140.451) (end 69.811 140.9435) (width 0.16) (layer "B.Cu") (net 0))
 (segment (start 71.1735 140.0785) (end 71.1735 139.9635) (width 0.16) (layer "B.Cu") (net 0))
 (segment (start 70.2835 136.5185) (end 69.7185 137.0835) (width 0.16) (layer "B.Cu") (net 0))
 (segment (start 90.7875 128.297) (end 89.7875 127.297) (width 0.16) (layer "B.Cu") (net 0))
 (segment (start 76.205931 140.1885) (end 75.77506 140.619371) (width 0.16) (layer "B.Cu") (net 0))
 (segment (start 84.6785 126.8135) (end 83.7885 125.9235) (width 0.16) (layer "B.Cu") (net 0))
 (segment (start 87.9485 139.5685) (end 87.2675 138.8875) (width 0.16) (layer "B.Cu") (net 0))
 (segment (start 83.7075 139.0825) (end 84.8785 140.2535) (width 0.16) (layer "B.Cu") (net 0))
 (segment (start 74.8485 140.1885) (end 74.8485 140.7385) (width 0.16) (layer "B.Cu") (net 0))
 (segment (start 69.7435 126.8735) (end 68.9535 126.0835) (width 0.16) (layer "B.Cu") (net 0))
 (segment (start 69.2875 134.297) (end 68.7875 134.297) (width 0.16) (layer "B.Cu") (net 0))
 (segment (start 85.82498 141.19998) (end 88.55202 141.19998) (width 0.16) (layer "B.Cu") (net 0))
 (segment (start 68.9535 126.0835) (end 68.0435 126.0835) (width 0.16) (layer "B.Cu") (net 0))
 (segment (start 81.3935 140.2785) (end 82.31498 141.19998) (width 0.16) (layer "B.Cu") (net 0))
 (segment (start 71.4335 126.1035) (end 71.5135 126.1835) (width 0.16) (layer "B.Cu") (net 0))
 (segment (start 70.2785 134.288) (end 69.7875 133.797) (width 0.16) (layer "B.Cu") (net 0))
 (segment (start 70.2835 136.5185) (end 70.2835 137.646) (width 0.16) (layer "B.Cu") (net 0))
 (segment (start 80.28202 141.19998) (end 81.2035 140.2785) (width 0.16) (layer "B.Cu") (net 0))
 (segment (start 82.8175 127.9295) (end 81.7615 126.8735) (width 0.16) (layer "B.Cu") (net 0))
 (segment (start 82.6185 126.5035) (end 82.6535 126.5035) (width 0.16) (layer "B.Cu") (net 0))
 (segment (start 73.0245 140.7335) (end 72.778 140.98) (width 0.16) (layer "B.Cu") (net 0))
 (segment (start 82.8485 140.1835) (end 83.4035 140.1835) (width 0.16) (layer "B.Cu") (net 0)))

